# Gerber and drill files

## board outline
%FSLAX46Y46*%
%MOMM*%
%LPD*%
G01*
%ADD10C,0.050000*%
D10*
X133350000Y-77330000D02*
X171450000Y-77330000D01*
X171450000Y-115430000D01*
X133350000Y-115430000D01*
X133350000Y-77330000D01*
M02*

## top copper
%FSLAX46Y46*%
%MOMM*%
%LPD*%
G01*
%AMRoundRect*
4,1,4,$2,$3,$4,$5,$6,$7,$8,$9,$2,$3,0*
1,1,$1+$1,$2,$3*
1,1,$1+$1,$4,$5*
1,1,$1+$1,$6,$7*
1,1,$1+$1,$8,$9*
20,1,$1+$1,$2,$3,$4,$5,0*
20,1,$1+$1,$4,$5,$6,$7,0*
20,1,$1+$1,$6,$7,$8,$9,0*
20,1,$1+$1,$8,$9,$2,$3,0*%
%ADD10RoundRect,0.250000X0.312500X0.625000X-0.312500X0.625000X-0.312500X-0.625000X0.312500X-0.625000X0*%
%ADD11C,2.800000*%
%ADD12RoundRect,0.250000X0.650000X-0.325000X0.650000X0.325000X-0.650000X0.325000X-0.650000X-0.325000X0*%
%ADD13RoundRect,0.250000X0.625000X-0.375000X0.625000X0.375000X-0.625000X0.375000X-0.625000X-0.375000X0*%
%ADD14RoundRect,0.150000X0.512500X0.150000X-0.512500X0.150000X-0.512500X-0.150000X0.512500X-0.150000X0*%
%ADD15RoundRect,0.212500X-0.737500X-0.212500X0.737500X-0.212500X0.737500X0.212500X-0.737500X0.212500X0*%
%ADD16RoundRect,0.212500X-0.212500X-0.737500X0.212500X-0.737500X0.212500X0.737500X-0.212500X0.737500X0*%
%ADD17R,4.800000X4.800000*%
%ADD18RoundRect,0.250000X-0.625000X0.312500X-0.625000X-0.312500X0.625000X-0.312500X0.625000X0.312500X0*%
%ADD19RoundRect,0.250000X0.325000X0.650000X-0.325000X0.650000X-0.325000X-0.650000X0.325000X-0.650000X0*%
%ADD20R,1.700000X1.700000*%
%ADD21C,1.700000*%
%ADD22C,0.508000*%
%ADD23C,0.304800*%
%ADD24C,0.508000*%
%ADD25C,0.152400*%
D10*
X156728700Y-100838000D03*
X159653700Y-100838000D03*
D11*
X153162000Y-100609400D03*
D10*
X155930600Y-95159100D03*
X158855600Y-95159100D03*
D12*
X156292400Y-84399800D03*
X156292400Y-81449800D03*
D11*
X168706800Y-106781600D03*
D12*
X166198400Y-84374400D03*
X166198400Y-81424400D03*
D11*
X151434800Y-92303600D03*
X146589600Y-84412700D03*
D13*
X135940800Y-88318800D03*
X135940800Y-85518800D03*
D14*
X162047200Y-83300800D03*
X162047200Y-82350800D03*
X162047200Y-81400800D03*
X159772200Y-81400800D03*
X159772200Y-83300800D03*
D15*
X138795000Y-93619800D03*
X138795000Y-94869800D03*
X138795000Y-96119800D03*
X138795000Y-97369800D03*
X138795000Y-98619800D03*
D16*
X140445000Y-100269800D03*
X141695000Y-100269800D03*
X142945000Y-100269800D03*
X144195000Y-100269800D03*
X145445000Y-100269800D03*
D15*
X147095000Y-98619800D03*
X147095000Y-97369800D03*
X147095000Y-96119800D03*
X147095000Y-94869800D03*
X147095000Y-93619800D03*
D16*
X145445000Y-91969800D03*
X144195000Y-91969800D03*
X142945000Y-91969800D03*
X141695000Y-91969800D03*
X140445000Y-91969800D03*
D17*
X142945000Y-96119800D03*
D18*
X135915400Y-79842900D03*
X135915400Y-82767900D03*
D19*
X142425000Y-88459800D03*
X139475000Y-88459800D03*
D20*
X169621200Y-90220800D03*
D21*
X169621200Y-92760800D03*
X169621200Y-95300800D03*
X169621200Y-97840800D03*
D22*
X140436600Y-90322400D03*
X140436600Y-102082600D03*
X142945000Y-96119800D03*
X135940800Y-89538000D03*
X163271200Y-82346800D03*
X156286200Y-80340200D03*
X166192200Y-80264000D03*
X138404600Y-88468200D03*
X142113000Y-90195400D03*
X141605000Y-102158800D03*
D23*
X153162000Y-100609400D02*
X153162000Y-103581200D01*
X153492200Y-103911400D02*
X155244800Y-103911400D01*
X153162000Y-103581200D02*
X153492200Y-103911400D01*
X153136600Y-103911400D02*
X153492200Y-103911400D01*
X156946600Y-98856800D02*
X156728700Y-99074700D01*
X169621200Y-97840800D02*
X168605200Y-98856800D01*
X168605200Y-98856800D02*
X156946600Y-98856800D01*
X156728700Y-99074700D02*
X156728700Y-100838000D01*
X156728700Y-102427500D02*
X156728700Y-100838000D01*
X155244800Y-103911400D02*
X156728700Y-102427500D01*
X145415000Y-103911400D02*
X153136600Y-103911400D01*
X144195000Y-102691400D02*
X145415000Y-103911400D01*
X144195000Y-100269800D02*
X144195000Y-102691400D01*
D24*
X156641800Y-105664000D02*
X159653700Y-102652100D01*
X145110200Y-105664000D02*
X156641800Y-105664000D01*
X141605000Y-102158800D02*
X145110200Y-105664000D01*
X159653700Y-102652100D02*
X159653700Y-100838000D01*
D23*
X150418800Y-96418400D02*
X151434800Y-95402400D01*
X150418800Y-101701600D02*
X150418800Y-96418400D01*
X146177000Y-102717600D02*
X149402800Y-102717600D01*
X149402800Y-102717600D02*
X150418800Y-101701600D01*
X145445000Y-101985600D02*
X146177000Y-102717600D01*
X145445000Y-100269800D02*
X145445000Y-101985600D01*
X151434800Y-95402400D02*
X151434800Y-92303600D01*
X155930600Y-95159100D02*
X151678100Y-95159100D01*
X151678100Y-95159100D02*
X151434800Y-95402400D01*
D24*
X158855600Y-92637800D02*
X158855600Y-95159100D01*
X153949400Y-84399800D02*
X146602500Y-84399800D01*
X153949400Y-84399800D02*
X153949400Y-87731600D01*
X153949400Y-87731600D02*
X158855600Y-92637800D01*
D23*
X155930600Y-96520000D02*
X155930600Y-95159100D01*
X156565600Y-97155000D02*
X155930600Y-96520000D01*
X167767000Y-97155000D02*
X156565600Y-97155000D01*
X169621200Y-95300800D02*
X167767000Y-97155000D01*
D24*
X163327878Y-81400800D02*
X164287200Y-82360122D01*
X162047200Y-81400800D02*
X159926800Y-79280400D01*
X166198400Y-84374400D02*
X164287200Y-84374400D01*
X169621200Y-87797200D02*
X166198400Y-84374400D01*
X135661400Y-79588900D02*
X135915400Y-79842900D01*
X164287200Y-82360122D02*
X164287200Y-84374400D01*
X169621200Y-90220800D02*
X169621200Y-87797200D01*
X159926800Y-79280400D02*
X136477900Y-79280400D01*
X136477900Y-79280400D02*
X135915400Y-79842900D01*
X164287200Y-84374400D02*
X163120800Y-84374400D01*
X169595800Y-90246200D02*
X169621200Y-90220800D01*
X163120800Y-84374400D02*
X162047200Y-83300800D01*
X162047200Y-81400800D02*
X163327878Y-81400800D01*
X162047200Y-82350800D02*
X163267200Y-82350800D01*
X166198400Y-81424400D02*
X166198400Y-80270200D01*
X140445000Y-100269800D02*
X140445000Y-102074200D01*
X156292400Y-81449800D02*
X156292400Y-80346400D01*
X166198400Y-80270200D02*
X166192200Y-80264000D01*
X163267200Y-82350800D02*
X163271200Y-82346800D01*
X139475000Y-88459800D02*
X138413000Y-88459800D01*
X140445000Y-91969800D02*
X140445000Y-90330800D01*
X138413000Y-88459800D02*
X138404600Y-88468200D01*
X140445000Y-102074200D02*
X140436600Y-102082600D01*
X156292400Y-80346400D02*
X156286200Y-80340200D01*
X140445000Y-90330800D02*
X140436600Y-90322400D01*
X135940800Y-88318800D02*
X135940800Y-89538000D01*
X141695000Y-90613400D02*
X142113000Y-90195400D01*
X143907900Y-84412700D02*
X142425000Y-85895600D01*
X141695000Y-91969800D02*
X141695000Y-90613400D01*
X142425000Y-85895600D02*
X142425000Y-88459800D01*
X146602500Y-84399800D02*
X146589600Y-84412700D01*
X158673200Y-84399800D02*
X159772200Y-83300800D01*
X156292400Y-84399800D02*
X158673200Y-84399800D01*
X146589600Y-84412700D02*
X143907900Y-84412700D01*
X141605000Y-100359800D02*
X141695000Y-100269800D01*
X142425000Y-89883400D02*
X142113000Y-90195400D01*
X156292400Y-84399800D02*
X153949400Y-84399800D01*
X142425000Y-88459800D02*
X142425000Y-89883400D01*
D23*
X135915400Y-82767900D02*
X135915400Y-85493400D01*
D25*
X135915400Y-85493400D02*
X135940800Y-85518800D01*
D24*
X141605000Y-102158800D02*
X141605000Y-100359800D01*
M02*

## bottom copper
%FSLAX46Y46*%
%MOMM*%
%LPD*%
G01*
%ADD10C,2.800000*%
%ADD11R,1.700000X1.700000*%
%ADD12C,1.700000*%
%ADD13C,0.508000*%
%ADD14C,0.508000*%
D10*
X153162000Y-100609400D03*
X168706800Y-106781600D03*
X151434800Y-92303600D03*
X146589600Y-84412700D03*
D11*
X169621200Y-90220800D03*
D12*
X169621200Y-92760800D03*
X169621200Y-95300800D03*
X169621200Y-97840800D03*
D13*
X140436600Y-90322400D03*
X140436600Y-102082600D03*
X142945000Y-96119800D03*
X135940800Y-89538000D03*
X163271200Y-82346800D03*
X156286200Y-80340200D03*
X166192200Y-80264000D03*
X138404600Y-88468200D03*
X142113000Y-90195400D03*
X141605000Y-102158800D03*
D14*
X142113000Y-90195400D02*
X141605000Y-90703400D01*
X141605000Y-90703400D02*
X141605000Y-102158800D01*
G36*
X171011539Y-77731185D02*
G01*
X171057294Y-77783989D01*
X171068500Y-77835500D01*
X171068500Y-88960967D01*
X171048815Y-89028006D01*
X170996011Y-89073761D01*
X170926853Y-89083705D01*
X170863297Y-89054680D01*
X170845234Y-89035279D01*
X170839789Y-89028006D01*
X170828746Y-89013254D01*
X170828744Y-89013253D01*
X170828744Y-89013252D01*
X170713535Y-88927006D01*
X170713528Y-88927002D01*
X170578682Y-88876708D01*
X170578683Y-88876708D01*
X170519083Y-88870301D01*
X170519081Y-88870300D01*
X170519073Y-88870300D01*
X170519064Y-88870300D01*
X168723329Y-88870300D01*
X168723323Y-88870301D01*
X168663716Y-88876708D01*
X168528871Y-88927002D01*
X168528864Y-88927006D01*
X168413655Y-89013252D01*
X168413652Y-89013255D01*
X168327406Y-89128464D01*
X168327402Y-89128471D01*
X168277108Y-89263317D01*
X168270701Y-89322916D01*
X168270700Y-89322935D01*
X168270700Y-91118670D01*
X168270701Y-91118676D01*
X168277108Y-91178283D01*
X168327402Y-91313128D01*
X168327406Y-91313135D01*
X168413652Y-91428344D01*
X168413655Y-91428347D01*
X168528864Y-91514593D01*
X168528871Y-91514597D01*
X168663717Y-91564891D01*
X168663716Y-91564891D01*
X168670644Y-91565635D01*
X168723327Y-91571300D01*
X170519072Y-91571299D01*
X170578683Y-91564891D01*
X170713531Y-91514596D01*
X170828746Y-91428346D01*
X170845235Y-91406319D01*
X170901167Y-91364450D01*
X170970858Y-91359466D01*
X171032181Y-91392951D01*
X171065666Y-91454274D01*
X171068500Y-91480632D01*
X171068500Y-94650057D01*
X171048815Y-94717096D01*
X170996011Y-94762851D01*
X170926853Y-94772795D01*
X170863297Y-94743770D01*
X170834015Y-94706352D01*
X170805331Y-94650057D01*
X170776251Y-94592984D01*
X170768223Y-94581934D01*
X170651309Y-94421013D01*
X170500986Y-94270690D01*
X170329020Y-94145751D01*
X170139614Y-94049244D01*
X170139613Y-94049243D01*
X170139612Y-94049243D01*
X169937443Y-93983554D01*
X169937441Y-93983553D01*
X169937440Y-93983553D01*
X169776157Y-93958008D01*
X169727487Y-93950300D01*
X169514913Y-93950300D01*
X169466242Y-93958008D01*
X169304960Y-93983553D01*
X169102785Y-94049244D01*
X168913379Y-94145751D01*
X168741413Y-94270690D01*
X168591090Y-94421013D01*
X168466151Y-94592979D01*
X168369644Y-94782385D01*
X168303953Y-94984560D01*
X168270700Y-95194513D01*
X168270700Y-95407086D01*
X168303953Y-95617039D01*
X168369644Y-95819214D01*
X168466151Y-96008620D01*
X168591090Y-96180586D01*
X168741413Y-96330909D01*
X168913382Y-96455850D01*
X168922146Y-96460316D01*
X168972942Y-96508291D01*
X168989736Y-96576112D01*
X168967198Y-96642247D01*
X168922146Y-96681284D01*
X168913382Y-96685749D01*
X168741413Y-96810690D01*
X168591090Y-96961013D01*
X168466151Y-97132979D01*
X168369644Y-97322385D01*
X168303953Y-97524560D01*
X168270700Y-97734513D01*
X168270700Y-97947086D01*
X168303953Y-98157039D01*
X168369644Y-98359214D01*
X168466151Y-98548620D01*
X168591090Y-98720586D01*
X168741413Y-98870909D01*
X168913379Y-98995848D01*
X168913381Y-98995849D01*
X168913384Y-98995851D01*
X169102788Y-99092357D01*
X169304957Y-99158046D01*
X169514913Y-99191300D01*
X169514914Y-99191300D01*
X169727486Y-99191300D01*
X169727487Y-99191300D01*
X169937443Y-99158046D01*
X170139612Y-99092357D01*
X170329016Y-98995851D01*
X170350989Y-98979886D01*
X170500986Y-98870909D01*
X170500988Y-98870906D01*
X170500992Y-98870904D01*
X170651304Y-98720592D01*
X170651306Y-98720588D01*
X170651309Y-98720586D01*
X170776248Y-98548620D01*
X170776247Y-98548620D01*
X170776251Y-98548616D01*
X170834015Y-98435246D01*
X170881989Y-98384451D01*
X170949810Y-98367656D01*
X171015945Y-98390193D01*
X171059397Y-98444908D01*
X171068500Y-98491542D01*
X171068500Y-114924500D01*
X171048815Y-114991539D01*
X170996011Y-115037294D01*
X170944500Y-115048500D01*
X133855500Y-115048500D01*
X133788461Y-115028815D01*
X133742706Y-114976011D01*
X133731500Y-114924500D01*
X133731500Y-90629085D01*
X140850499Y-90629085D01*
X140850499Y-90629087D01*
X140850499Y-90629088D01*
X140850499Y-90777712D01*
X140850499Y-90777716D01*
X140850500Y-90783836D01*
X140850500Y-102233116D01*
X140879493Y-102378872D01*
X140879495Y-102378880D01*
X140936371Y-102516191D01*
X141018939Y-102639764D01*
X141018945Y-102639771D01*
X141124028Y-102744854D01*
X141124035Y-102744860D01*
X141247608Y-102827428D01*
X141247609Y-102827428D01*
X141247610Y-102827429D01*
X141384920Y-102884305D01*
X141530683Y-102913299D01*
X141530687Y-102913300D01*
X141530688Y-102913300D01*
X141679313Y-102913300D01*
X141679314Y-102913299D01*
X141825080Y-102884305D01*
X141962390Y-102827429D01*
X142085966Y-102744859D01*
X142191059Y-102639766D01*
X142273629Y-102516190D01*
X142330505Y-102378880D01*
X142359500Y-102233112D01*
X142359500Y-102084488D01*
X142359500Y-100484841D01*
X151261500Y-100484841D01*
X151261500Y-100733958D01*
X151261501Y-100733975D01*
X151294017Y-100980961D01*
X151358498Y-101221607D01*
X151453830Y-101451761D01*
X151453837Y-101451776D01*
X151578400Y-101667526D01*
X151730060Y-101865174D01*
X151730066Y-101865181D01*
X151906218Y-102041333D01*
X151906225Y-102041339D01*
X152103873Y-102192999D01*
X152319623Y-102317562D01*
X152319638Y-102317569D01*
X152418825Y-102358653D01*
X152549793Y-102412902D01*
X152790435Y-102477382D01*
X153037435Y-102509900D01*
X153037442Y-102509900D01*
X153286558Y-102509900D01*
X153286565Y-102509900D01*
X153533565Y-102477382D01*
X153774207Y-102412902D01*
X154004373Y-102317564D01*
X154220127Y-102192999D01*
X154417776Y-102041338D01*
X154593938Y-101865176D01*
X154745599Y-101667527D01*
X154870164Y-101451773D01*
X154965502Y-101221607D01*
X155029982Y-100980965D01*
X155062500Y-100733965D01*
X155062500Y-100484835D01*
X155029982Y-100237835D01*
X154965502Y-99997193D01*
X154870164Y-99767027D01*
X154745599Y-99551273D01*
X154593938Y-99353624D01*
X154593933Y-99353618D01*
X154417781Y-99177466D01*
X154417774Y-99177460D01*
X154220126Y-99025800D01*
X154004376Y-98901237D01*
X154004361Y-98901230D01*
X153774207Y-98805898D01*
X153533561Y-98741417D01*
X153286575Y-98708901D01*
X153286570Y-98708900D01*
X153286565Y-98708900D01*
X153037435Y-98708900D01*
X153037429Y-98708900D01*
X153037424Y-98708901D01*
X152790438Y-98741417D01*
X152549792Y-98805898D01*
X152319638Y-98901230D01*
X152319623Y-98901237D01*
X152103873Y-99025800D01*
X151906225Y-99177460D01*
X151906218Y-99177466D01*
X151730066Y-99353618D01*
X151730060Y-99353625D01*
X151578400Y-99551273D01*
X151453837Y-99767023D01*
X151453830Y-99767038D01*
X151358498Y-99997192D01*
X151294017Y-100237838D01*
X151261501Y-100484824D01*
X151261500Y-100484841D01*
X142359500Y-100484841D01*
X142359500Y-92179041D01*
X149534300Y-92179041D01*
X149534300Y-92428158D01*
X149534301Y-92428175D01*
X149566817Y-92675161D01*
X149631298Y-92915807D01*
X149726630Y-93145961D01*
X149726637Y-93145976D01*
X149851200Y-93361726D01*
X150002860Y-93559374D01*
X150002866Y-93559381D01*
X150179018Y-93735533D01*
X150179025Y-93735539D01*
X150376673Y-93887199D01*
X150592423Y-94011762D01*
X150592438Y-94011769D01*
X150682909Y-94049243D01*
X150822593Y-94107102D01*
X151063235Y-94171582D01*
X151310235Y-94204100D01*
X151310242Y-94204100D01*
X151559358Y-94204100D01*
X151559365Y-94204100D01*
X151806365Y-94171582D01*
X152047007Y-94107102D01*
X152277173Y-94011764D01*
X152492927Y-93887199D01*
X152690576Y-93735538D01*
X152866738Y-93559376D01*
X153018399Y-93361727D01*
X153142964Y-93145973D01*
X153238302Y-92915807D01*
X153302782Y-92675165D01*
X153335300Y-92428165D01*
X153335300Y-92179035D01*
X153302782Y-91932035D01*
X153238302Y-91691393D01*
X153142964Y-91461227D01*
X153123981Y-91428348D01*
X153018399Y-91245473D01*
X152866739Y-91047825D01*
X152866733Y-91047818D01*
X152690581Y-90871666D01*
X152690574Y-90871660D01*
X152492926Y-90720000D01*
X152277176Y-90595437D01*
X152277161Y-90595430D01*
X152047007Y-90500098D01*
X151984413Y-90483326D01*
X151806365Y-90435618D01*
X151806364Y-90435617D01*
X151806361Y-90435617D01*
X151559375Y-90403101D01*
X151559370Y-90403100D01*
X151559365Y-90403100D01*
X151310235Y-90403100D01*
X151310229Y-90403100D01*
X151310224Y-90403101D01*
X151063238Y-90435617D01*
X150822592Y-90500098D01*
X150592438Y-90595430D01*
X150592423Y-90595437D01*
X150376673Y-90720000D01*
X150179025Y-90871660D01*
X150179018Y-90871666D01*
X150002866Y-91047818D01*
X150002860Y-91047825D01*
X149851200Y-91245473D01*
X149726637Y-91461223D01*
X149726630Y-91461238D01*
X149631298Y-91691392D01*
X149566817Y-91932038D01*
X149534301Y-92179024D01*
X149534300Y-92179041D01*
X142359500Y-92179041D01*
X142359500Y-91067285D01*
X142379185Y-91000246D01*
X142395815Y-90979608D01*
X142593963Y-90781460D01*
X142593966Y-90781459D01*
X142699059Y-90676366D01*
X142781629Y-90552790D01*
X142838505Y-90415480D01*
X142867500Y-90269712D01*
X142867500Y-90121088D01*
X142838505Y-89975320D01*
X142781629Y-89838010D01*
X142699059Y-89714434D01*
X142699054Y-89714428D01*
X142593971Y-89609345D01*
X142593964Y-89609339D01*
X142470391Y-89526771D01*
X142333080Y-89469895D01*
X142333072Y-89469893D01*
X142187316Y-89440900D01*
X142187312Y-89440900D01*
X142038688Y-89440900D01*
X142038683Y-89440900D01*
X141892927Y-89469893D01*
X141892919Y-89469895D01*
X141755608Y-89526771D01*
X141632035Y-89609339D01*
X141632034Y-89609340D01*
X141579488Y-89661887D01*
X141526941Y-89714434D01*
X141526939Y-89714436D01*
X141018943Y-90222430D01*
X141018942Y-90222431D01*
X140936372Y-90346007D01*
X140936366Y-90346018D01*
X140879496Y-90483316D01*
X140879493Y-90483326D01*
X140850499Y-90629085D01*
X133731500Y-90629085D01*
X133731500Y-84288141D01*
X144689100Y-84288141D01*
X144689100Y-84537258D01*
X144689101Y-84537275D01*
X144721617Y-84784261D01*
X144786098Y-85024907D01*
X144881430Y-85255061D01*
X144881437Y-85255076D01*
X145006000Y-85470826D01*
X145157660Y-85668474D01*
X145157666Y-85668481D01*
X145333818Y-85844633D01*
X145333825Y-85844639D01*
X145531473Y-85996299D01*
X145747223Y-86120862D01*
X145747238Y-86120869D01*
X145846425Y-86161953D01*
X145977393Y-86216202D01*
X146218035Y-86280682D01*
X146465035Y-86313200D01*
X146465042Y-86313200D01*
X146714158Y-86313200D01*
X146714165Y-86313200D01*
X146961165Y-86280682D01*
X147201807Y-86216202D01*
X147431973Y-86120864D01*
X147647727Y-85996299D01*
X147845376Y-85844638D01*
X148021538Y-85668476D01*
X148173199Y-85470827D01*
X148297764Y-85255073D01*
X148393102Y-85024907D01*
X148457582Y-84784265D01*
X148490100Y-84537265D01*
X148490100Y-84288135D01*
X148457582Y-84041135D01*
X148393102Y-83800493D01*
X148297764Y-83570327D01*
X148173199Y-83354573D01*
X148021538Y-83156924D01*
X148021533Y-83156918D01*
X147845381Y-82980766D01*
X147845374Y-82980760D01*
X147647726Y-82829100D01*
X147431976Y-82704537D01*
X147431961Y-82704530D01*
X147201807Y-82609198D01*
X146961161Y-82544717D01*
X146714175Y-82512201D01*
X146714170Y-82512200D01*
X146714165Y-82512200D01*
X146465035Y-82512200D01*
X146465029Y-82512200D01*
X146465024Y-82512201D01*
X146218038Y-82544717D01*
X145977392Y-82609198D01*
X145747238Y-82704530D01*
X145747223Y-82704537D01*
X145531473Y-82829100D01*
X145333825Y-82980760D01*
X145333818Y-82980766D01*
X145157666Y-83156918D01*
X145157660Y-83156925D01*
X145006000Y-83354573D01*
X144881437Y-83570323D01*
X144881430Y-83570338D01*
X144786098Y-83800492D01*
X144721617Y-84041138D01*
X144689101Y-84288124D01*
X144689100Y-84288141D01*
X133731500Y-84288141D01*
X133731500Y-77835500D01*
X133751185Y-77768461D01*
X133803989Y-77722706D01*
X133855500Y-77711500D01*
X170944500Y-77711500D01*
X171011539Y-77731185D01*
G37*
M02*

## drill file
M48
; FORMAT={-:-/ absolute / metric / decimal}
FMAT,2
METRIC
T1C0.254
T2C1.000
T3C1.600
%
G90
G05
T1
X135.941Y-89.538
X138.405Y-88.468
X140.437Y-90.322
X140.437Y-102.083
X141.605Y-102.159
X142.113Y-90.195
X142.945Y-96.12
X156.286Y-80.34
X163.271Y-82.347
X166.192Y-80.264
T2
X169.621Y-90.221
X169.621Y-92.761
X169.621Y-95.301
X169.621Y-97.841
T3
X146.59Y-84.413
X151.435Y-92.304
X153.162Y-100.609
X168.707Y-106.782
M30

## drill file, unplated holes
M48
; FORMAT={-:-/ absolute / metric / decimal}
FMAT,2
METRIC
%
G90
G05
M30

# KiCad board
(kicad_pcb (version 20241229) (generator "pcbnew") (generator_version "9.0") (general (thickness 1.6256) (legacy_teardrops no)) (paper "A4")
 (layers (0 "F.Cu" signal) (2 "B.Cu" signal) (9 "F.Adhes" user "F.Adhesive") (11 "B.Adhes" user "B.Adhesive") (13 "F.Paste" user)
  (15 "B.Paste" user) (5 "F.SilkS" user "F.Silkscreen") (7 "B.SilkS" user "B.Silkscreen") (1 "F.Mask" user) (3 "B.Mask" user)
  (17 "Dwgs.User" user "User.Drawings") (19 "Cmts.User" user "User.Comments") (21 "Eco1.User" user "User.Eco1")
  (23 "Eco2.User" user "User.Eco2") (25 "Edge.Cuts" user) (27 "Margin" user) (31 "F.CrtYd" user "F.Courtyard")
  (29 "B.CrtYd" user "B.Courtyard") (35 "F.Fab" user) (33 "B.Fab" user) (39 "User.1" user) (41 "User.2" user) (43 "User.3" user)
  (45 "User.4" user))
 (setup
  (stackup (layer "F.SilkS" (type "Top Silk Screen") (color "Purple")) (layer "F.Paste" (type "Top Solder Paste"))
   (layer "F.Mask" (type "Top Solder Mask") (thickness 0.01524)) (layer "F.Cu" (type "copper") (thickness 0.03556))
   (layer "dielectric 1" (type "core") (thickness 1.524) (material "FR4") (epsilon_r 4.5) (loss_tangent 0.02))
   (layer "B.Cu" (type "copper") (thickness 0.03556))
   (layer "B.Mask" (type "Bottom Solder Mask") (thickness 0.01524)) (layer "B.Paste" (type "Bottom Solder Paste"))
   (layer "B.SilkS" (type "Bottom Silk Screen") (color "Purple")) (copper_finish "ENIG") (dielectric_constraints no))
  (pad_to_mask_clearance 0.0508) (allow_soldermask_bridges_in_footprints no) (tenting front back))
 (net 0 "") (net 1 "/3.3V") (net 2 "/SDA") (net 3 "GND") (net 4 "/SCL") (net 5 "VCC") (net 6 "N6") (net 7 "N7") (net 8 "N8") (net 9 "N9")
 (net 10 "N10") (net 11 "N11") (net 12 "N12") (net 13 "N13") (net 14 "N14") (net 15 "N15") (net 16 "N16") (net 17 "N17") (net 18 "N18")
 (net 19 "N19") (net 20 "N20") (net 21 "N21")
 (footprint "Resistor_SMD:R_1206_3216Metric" (layer "F.Cu") (at 157.3931 95.1591 180)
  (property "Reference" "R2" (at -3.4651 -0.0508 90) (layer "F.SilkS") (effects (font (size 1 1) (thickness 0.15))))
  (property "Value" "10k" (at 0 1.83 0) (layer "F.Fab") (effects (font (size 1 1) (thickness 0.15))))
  (pad "1" smd roundrect (at -1.4625 0 180) (size 1.125 1.75) (layers "F.Cu" "F.Mask" "F.Paste") (roundrect_rratio 0.222222) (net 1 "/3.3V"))
  (pad "2" smd roundrect (at 1.4625 0 180) (size 1.125 1.75) (layers "F.Cu" "F.Mask" "F.Paste") (roundrect_rratio 0.222222) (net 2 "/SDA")))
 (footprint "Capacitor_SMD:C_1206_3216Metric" (layer "F.Cu") (at 156.2924 82.9248 90)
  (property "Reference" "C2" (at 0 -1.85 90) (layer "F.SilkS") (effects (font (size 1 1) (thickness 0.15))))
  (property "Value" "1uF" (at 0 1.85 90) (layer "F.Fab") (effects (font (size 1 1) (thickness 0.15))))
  (pad "1" smd roundrect (at -1.475 0 90) (size 1.15 1.8) (layers "F.Cu" "F.Mask" "F.Paste") (roundrect_rratio 0.217391) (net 1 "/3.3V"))
  (pad "2" smd roundrect (at 1.475 0 90) (size 1.15 1.8) (layers "F.Cu" "F.Mask" "F.Paste") (roundrect_rratio 0.217391) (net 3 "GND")))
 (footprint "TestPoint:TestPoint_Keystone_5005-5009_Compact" (layer "F.Cu") (at 153.162 100.6094)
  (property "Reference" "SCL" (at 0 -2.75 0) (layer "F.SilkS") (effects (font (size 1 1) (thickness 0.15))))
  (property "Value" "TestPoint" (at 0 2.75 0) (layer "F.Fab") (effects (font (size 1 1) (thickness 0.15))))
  (pad "1" thru_hole circle (at 0 0) (size 2.8 2.8) (drill 1.6) (layers "*.Cu" "*.Mask") (remove_unused_layers no) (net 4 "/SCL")))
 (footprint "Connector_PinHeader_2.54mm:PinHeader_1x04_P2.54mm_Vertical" (layer "F.Cu") (at 169.6212 90.2208)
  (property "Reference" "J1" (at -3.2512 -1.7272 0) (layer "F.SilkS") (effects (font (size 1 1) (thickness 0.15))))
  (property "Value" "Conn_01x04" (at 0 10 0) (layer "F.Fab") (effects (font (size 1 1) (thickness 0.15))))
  (pad "1" thru_hole rect (at 0 0) (size 1.7 1.7) (drill 1) (layers "*.Cu" "*.Mask") (remove_unused_layers no) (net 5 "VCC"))
  (pad "2" thru_hole circle (at 0 2.54) (size 1.7 1.7) (drill 1) (layers "*.Cu" "*.Mask") (remove_unused_layers no) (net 3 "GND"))
  (pad "3" thru_hole circle (at 0 5.08) (size 1.7 1.7) (drill 1) (layers "*.Cu" "*.Mask") (remove_unused_layers no) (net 2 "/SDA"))
  (pad "4" thru_hole circle (at 0 7.62) (size 1.7 1.7) (drill 1) (layers "*.Cu" "*.Mask") (remove_unused_layers no) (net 4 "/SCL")))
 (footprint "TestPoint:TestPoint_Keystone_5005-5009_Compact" (layer "F.Cu") (at 168.7068 106.7816)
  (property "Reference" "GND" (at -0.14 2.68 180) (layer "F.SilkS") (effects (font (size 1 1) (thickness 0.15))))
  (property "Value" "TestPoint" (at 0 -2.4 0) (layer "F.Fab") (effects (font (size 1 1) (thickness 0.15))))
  (pad "1" thru_hole circle (at 0 0) (size 2.8 2.8) (drill 1.6) (layers "*.Cu" "*.Mask") (remove_unused_layers no) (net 3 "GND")))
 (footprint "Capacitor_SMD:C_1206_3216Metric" (layer "F.Cu") (at 166.1984 82.8994 90)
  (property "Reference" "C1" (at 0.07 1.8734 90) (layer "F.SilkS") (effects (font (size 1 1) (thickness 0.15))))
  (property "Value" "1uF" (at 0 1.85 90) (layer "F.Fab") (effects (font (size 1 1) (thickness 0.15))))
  (pad "1" smd roundrect (at -1.475 0 90) (size 1.15 1.8) (layers "F.Cu" "F.Mask" "F.Paste") (roundrect_rratio 0.217391) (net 5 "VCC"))
  (pad "2" smd roundrect (at 1.475 0 90) (size 1.15 1.8) (layers "F.Cu" "F.Mask" "F.Paste") (roundrect_rratio 0.217391) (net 3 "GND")))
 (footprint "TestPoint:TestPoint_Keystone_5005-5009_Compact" (layer "F.Cu") (at 151.4348 92.3036)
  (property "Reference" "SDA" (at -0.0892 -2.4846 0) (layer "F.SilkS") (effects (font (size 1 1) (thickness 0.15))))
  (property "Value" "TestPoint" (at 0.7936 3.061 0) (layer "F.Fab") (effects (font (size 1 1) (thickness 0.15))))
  (pad "1" thru_hole circle (at 0 0) (size 2.8 2.8) (drill 1.6) (layers "*.Cu" "*.Mask") (remove_unused_layers no) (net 2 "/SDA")))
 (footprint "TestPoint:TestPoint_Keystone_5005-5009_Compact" (layer "F.Cu") (at 146.5896 84.4127)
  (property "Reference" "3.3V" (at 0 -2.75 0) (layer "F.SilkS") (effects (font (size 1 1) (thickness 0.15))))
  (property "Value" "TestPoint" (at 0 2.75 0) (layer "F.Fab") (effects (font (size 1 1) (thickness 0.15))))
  (pad "1" thru_hole circle (at 0 0) (size 2.8 2.8) (drill 1.6) (layers "*.Cu" "*.Mask") (remove_unused_layers no) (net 1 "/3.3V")))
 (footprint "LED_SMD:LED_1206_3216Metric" (layer "F.Cu") (at 135.9408 86.9188 90)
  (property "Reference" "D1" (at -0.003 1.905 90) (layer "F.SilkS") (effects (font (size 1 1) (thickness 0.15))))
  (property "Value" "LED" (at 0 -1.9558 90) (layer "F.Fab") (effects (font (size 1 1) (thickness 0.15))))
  (pad "1" smd roundrect (at -1.4 0 90) (size 1.25 1.75) (layers "F.Cu" "F.Mask" "F.Paste") (roundrect_rratio 0.2) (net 3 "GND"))
  (pad "2" smd roundrect (at 1.4 0 90) (size 1.25 1.75) (layers "F.Cu" "F.Mask" "F.Paste") (roundrect_rratio 0.2) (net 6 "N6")))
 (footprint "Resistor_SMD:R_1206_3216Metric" (layer "F.Cu") (at 158.1912 100.838 180)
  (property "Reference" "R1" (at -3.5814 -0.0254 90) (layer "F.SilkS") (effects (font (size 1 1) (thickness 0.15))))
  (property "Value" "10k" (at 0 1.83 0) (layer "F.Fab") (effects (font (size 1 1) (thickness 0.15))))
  (pad "1" smd roundrect (at -1.4625 0 180) (size 1.125 1.75) (layers "F.Cu" "F.Mask" "F.Paste") (roundrect_rratio 0.222222) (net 1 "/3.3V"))
  (pad "2" smd roundrect (at 1.4625 0 180) (size 1.125 1.75) (layers "F.Cu" "F.Mask" "F.Paste") (roundrect_rratio 0.222222) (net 4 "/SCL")))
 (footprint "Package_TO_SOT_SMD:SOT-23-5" (layer "F.Cu") (at 160.9097 82.3508 180)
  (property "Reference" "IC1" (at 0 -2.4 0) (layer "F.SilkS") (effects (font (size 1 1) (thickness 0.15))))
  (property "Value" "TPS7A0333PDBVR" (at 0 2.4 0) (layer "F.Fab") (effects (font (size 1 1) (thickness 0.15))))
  (pad "1" smd roundrect (at -1.1375 -0.95 180) (size 1.325 0.6) (layers "F.Cu" "F.Mask" "F.Paste") (roundrect_rratio 0.25) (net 5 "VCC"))
  (pad "2" smd roundrect (at -1.1375 0 180) (size 1.325 0.6) (layers "F.Cu" "F.Mask" "F.Paste") (roundrect_rratio 0.25) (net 3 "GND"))
  (pad "3" smd roundrect (at -1.1375 0.95 180) (size 1.325 0.6) (layers "F.Cu" "F.Mask" "F.Paste") (roundrect_rratio 0.25) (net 5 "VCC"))
  (pad "4" smd roundrect (at 1.1375 0.95 180) (size 1.325 0.6) (layers "F.Cu" "F.Mask" "F.Paste") (roundrect_rratio 0.25) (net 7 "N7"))
  (pad "5" smd roundrect (at 1.1375 -0.95 180) (size 1.325 0.6) (layers "F.Cu" "F.Mask" "F.Paste") (roundrect_rratio 0.25) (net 1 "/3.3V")))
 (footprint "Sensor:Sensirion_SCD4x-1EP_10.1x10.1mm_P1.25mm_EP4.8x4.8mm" (layer "F.Cu") (at 142.945 96.1198)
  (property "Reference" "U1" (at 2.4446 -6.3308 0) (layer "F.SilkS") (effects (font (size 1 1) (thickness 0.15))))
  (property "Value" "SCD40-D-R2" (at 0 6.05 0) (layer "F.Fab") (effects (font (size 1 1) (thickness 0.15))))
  (pad "" smd roundrect (at -1.2 -1.2) (size 1.93 1.93) (layers "F.Paste") (roundrect_rratio 0.129534))
  (pad "" smd roundrect (at -1.2 1.2) (size 1.93 1.93) (layers "F.Paste") (roundrect_rratio 0.129534))
  (pad "" smd roundrect (at 1.2 -1.2) (size 1.93 1.93) (layers "F.Paste") (roundrect_rratio 0.129534))
  (pad "" smd roundrect (at 1.2 1.2) (size 1.93 1.93) (layers "F.Paste") (roundrect_rratio 0.129534))
  (pad "1" smd roundrect (at -4.15 -2.5) (size 1.9 0.85) (layers "F.Cu" "F.Mask" "F.Paste") (roundrect_rratio 0.25) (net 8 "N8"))
  (pad "2" smd roundrect (at -4.15 -1.25) (size 1.9 0.85) (layers "F.Cu" "F.Mask" "F.Paste") (roundrect_rratio 0.25) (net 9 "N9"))
  (pad "3" smd roundrect (at -4.15 0) (size 1.9 0.85) (layers "F.Cu" "F.Mask" "F.Paste") (roundrect_rratio 0.25) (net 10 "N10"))
  (pad "4" smd roundrect (at -4.15 1.25) (size 1.9 0.85) (layers "F.Cu" "F.Mask" "F.Paste") (roundrect_rratio 0.25) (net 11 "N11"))
  (pad "5" smd roundrect (at -4.15 2.5) (size 1.9 0.85) (layers "F.Cu" "F.Mask" "F.Paste") (roundrect_rratio 0.25) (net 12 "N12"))
  (pad "6" smd roundrect (at -2.5 4.15) (size 0.85 1.9) (layers "F.Cu" "F.Mask" "F.Paste") (roundrect_rratio 0.25) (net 3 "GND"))
  (pad "7" smd roundrect (at -1.25 4.15) (size 0.85 1.9) (layers "F.Cu" "F.Mask" "F.Paste") (roundrect_rratio 0.25) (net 1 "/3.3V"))
  (pad "8" smd roundrect (at 0 4.15) (size 0.85 1.9) (layers "F.Cu" "F.Mask" "F.Paste") (roundrect_rratio 0.25) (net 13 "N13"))
  (pad "9" smd roundrect (at 1.25 4.15) (size 0.85 1.9) (layers "F.Cu" "F.Mask" "F.Paste") (roundrect_rratio 0.25) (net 4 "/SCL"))
  (pad "10" smd roundrect (at 2.5 4.15) (size 0.85 1.9) (layers "F.Cu" "F.Mask" "F.Paste") (roundrect_rratio 0.25) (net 2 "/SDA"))
  (pad "11" smd roundrect (at 4.15 2.5) (size 1.9 0.85) (layers "F.Cu" "F.Mask" "F.Paste") (roundrect_rratio 0.25) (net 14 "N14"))
  (pad "12" smd roundrect (at 4.15 1.25) (size 1.9 0.85) (layers "F.Cu" "F.Mask" "F.Paste") (roundrect_rratio 0.25) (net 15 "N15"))
  (pad "13" smd roundrect (at 4.15 0) (size 1.9 0.85) (layers "F.Cu" "F.Mask" "F.Paste") (roundrect_rratio 0.25) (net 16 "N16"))
  (pad "14" smd roundrect (at 4.15 -1.25) (size 1.9 0.85) (layers "F.Cu" "F.Mask" "F.Paste") (roundrect_rratio 0.25) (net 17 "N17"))
  (pad "15" smd roundrect (at 4.15 -2.5) (size 1.9 0.85) (layers "F.Cu" "F.Mask" "F.Paste") (roundrect_rratio 0.25) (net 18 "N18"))
  (pad "16" smd roundrect (at 2.5 -4.15) (size 0.85 1.9) (layers "F.Cu" "F.Mask" "F.Paste") (roundrect_rratio 0.25) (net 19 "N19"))
  (pad "17" smd roundrect (at 1.25 -4.15) (size 0.85 1.9) (layers "F.Cu" "F.Mask" "F.Paste") (roundrect_rratio 0.25) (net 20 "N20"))
  (pad "18" smd roundrect (at 0 -4.15) (size 0.85 1.9) (layers "F.Cu" "F.Mask" "F.Paste") (roundrect_rratio 0.25) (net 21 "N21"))
  (pad "19" smd roundrect (at -1.25 -4.15) (size 0.85 1.9) (layers "F.Cu" "F.Mask" "F.Paste") (roundrect_rratio 0.25) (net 1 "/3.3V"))
  (pad "20" smd roundrect (at -2.5 -4.15) (size 0.85 1.9) (layers "F.Cu" "F.Mask" "F.Paste") (roundrect_rratio 0.25) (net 3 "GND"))
  (pad "21" smd rect (at 0 0) (size 4.8 4.8) (layers "F.Cu" "F.Mask") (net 3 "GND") (zone_connect 2)))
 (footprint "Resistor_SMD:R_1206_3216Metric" (layer "F.Cu") (at 135.9154 81.3054 -90)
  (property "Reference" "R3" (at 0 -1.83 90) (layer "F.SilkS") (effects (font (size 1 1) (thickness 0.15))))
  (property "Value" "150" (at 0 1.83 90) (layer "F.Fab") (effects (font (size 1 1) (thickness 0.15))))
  (pad "1" smd roundrect (at -1.4625 0 270) (size 1.125 1.75) (layers "F.Cu" "F.Mask" "F.Paste") (roundrect_rratio 0.222222) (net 5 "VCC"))
  (pad "2" smd roundrect (at 1.4625 0 270) (size 1.125 1.75) (layers "F.Cu" "F.Mask" "F.Paste") (roundrect_rratio 0.222222) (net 6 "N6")))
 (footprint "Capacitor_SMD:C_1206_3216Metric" (layer "F.Cu") (at 140.95 88.4598 180)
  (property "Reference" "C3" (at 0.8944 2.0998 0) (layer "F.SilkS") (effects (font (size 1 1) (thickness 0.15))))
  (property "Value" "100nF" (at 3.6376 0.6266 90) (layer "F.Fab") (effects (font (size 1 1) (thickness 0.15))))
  (pad "1" smd roundrect (at -1.475 0 180) (size 1.15 1.8) (layers "F.Cu" "F.Mask" "F.Paste") (roundrect_rratio 0.217391) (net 1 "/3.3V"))
  (pad "2" smd roundrect (at 1.475 0 180) (size 1.15 1.8) (layers "F.Cu" "F.Mask" "F.Paste") (roundrect_rratio 0.217391) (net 3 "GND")))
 (gr_rect (start 133.35 77.33) (end 171.45 115.43) (stroke (width 0.05) (type default)) (fill no) (layer "Edge.Cuts"))
 (segment (start 163.327878 81.4008) (end 164.2872 82.360122) (width 0.508) (layer "F.Cu") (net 5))
 (segment (start 162.0472 81.4008) (end 159.9268 79.2804) (width 0.508) (layer "F.Cu") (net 5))
 (segment (start 166.1984 84.3744) (end 164.2872 84.3744) (width 0.508) (layer "F.Cu") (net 5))
 (segment (start 169.6212 87.7972) (end 166.1984 84.3744) (width 0.508) (layer "F.Cu") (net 5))
 (segment (start 135.6614 79.5889) (end 135.9154 79.8429) (width 0.508) (layer "F.Cu") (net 5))
 (segment (start 164.2872 82.360122) (end 164.2872 84.3744) (width 0.508) (layer "F.Cu") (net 5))
 (segment (start 169.6212 90.2208) (end 169.6212 87.7972) (width 0.508) (layer "F.Cu") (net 5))
 (segment (start 159.9268 79.2804) (end 136.4779 79.2804) (width 0.508) (layer "F.Cu") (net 5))
 (segment (start 136.4779 79.2804) (end 135.9154 79.8429) (width 0.508) (layer "F.Cu") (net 5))
 (segment (start 164.2872 84.3744) (end 163.1208 84.3744) (width 0.508) (layer "F.Cu") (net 5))
 (segment (start 169.5958 90.2462) (end 169.6212 90.2208) (width 0.508) (layer "F.Cu") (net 5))
 (segment (start 163.1208 84.3744) (end 162.0472 83.3008) (width 0.508) (layer "F.Cu") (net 5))
 (segment (start 162.0472 81.4008) (end 163.327878 81.4008) (width 0.508) (layer "F.Cu") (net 5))
 (segment (start 162.0472 82.3508) (end 163.2672 82.3508) (width 0.508) (layer "F.Cu") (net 3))
 (segment (start 166.1984 81.4244) (end 166.1984 80.2702) (width 0.508) (layer "F.Cu") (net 3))
 (segment (start 140.445 100.2698) (end 140.445 102.0742) (width 0.508) (layer "F.Cu") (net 3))
 (segment (start 156.2924 81.4498) (end 156.2924 80.3464) (width 0.508) (layer "F.Cu") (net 3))
 (segment (start 166.1984 80.2702) (end 166.1922 80.264) (width 0.508) (layer "F.Cu") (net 3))
 (segment (start 163.2672 82.3508) (end 163.2712 82.3468) (width 0.508) (layer "F.Cu") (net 3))
 (segment (start 139.475 88.4598) (end 138.413 88.4598) (width 0.508) (layer "F.Cu") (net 3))
 (segment (start 140.445 91.9698) (end 140.445 90.3308) (width 0.508) (layer "F.Cu") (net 3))
 (segment (start 138.413 88.4598) (end 138.4046 88.4682) (width 0.508) (layer "F.Cu") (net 3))
 (segment (start 140.445 102.0742) (end 140.4366 102.0826) (width 0.508) (layer "F.Cu") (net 3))
 (segment (start 156.2924 80.3464) (end 156.2862 80.3402) (width 0.508) (layer "F.Cu") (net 3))
 (segment (start 140.445 90.3308) (end 140.4366 90.3224) (width 0.508) (layer "F.Cu") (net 3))
 (segment (start 135.9408 88.3188) (end 135.9408 89.538) (width 0.508) (layer "F.Cu") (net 3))
 (via (at 140.4366 90.3224) (size 0.508) (drill 0.254) (layers "F.Cu" "B.Cu") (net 3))
 (via (at 140.4366 102.0826) (size 0.508) (drill 0.254) (layers "F.Cu" "B.Cu") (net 3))
 (via (at 142.945 96.1198) (size 0.508) (drill 0.254) (layers "F.Cu" "B.Cu") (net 3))
 (via (at 135.9408 89.538) (size 0.508) (drill 0.254) (layers "F.Cu" "B.Cu") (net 3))
 (via (at 163.2712 82.3468) (size 0.508) (drill 0.254) (layers "F.Cu" "B.Cu") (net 3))
 (via (at 156.2862 80.3402) (size 0.508) (drill 0.254) (layers "F.Cu" "B.Cu") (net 3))
 (via (at 166.1922 80.264) (size 0.508) (drill 0.254) (layers "F.Cu" "B.Cu") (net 3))
 (via (at 138.4046 88.4682) (size 0.508) (drill 0.254) (layers "F.Cu" "B.Cu") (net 3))
 (segment (start 159.6537 102.6521) (end 159.6537 100.838) (width 0.508) (layer "F.Cu") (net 1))
 (segment (start 141.695 90.6134) (end 142.113 90.1954) (width 0.508) (layer "F.Cu") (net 1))
 (segment (start 143.9079 84.4127) (end 142.425 85.8956) (width 0.508) (layer "F.Cu") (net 1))
 (segment (start 153.9494 84.3998) (end 146.6025 84.3998) (width 0.508) (layer "F.Cu") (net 1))
 (segment (start 141.695 91.9698) (end 141.695 90.6134) (width 0.508) (layer "F.Cu") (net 1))
 (segment (start 142.425 85.8956) (end 142.425 88.4598) (width 0.508) (layer "F.Cu") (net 1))
 (segment (start 156.6418 105.664) (end 159.6537 102.6521) (width 0.508) (layer "F.Cu") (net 1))
 (segment (start 146.6025 84.3998) (end 146.5896 84.4127) (width 0.508) (layer "F.Cu") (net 1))
 (segment (start 158.6732 84.3998) (end 159.7722 83.3008) (width 0.508) (layer "F.Cu") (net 1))
 (segment (start 141.605 102.1588) (end 145.1102 105.664) (width 0.508) (layer "F.Cu") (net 1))
 (segment (start 145.1102 105.664) (end 156.6418 105.664) (width 0.508) (layer "F.Cu") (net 1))
 (segment (start 153.9494 84.3998) (end 153.9494 87.7316) (width 0.508) (layer "F.Cu") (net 1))
 (segment (start 156.2924 84.3998) (end 158.6732 84.3998) (width 0.508) (layer "F.Cu") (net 1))
 (segment (start 146.5896 84.4127) (end 143.9079 84.4127) (width 0.508) (layer "F.Cu") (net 1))
 (segment (start 141.605 100.3598) (end 141.695 100.2698) (width 0.508) (layer "F.Cu") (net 1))
 (segment (start 142.425 89.8834) (end 142.113 90.1954) (width 0.508) (layer "F.Cu") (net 1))
 (segment (start 156.2924 84.3998) (end 153.9494 84.3998) (width 0.508) (layer "F.Cu") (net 1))
 (segment (start 141.605 102.1588) (end 141.605 100.3598) (width 0.508) (layer "F.Cu") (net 1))
 (segment (start 158.8556 92.6378) (end 158.8556 95.1591) (width 0.508) (layer "F.Cu") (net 1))
 (segment (start 142.425 88.4598) (end 142.425 89.8834) (width 0.508) (layer "F.Cu") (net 1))
 (segment (start 153.9494 87.7316) (end 158.8556 92.6378) (width 0.508) (layer "F.Cu") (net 1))
 (via (at 141.605 102.1588) (size 0.508) (drill 0.254) (layers "F.Cu" "B.Cu") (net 1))
 (via (at 142.113 90.1954) (size 0.508) (drill 0.254) (layers "F.Cu" "B.Cu") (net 1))
 (segment (start 142.113 90.1954) (end 141.605 90.7034) (width 0.508) (layer "B.Cu") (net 1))
 (segment (start 141.605 90.7034) (end 141.605 102.1588) (width 0.508) (layer "B.Cu") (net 1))
 (segment (start 135.9154 82.7679) (end 135.9154 85.4934) (width 0.3048) (layer "F.Cu") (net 6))
 (segment (start 135.9154 85.4934) (end 135.9408 85.5188) (width 0.1524) (layer "F.Cu") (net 6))
 (segment (start 156.7287 102.4275) (end 156.7287 100.838) (width 0.3048) (layer "F.Cu") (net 4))
 (segment (start 155.2448 103.9114) (end 156.7287 102.4275) (width 0.3048) (layer "F.Cu") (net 4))
 (segment (start 144.195 102.6914) (end 145.415 103.9114) (width 0.3048) (layer "F.Cu") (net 4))
 (segment (start 153.4922 103.9114) (end 155.2448 103.9114) (width 0.3048) (layer "F.Cu") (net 4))
 (segment (start 156.7287 99.0747) (end 156.7287 100.838) (width 0.3048) (layer "F.Cu") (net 4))
 (segment (start 153.162 103.5812) (end 153.4922 103.9114) (width 0.3048) (layer "F.Cu") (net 4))
 (segment (start 145.415 103.9114) (end 153.1366 103.9114) (width 0.3048) (layer "F.Cu") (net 4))
 (segment (start 153.1366 103.9114) (end 153.4922 103.9114) (width 0.3048) (layer "F.Cu") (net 4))
 (segment (start 144.195 100.2698) (end 144.195 102.6914) (width 0.3048) (layer "F.Cu") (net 4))
 (segment (start 169.6212 97.8408) (end 168.6052 98.8568) (width 0.3048) (layer "F.Cu") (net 4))
 (segment (start 156.9466 98.8568) (end 156.7287 99.0747) (width 0.3048) (layer "F.Cu") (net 4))
 (segment (start 168.6052 98.8568) (end 156.9466 98.8568) (width 0.3048) (layer "F.Cu") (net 4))
 (segment (start 153.162 100.6094) (end 153.162 103.5812) (width 0.3048) (layer "F.Cu") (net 4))
 (segment (start 167.767 97.155) (end 156.5656 97.155) (width 0.3048) (layer "F.Cu") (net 2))
 (segment (start 145.445 100.2698) (end 145.445 101.9856) (width 0.3048) (layer "F.Cu") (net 2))
 (segment (start 155.9306 96.52) (end 155.9306 95.1591) (width 0.3048) (layer "F.Cu") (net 2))
 (segment (start 150.4188 96.4184) (end 151.4348 95.4024) (width 0.3048) (layer "F.Cu") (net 2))
 (segment (start 145.445 101.9856) (end 146.177 102.7176) (width 0.3048) (layer "F.Cu") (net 2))
 (segment (start 149.4028 102.7176) (end 150.4188 101.7016) (width 0.3048) (layer "F.Cu") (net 2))
 (segment (start 169.6212 95.3008) (end 167.767 97.155) (width 0.3048) (layer "F.Cu") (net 2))
 (segment (start 146.177 102.7176) (end 149.4028 102.7176) (width 0.3048) (layer "F.Cu") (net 2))
 (segment (start 151.4348 95.4024) (end 151.4348 92.3036) (width 0.3048) (layer "F.Cu") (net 2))
 (segment (start 150.4188 101.7016) (end 150.4188 96.4184) (width 0.3048) (layer "F.Cu") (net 2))
 (segment (start 151.6781 95.1591) (end 151.4348 95.4024) (width 0.3048) (layer "F.Cu") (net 2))
 (segment (start 156.5656 97.155) (end 155.9306 96.52) (width 0.3048) (layer "F.Cu") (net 2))
 (segment (start 155.9306 95.1591) (end 151.6781 95.1591) (width 0.3048) (layer "F.Cu") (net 2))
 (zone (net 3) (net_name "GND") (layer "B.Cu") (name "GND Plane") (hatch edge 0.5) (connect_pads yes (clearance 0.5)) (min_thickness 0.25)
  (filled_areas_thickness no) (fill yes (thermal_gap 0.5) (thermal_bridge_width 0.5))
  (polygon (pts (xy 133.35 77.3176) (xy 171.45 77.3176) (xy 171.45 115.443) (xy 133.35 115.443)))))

